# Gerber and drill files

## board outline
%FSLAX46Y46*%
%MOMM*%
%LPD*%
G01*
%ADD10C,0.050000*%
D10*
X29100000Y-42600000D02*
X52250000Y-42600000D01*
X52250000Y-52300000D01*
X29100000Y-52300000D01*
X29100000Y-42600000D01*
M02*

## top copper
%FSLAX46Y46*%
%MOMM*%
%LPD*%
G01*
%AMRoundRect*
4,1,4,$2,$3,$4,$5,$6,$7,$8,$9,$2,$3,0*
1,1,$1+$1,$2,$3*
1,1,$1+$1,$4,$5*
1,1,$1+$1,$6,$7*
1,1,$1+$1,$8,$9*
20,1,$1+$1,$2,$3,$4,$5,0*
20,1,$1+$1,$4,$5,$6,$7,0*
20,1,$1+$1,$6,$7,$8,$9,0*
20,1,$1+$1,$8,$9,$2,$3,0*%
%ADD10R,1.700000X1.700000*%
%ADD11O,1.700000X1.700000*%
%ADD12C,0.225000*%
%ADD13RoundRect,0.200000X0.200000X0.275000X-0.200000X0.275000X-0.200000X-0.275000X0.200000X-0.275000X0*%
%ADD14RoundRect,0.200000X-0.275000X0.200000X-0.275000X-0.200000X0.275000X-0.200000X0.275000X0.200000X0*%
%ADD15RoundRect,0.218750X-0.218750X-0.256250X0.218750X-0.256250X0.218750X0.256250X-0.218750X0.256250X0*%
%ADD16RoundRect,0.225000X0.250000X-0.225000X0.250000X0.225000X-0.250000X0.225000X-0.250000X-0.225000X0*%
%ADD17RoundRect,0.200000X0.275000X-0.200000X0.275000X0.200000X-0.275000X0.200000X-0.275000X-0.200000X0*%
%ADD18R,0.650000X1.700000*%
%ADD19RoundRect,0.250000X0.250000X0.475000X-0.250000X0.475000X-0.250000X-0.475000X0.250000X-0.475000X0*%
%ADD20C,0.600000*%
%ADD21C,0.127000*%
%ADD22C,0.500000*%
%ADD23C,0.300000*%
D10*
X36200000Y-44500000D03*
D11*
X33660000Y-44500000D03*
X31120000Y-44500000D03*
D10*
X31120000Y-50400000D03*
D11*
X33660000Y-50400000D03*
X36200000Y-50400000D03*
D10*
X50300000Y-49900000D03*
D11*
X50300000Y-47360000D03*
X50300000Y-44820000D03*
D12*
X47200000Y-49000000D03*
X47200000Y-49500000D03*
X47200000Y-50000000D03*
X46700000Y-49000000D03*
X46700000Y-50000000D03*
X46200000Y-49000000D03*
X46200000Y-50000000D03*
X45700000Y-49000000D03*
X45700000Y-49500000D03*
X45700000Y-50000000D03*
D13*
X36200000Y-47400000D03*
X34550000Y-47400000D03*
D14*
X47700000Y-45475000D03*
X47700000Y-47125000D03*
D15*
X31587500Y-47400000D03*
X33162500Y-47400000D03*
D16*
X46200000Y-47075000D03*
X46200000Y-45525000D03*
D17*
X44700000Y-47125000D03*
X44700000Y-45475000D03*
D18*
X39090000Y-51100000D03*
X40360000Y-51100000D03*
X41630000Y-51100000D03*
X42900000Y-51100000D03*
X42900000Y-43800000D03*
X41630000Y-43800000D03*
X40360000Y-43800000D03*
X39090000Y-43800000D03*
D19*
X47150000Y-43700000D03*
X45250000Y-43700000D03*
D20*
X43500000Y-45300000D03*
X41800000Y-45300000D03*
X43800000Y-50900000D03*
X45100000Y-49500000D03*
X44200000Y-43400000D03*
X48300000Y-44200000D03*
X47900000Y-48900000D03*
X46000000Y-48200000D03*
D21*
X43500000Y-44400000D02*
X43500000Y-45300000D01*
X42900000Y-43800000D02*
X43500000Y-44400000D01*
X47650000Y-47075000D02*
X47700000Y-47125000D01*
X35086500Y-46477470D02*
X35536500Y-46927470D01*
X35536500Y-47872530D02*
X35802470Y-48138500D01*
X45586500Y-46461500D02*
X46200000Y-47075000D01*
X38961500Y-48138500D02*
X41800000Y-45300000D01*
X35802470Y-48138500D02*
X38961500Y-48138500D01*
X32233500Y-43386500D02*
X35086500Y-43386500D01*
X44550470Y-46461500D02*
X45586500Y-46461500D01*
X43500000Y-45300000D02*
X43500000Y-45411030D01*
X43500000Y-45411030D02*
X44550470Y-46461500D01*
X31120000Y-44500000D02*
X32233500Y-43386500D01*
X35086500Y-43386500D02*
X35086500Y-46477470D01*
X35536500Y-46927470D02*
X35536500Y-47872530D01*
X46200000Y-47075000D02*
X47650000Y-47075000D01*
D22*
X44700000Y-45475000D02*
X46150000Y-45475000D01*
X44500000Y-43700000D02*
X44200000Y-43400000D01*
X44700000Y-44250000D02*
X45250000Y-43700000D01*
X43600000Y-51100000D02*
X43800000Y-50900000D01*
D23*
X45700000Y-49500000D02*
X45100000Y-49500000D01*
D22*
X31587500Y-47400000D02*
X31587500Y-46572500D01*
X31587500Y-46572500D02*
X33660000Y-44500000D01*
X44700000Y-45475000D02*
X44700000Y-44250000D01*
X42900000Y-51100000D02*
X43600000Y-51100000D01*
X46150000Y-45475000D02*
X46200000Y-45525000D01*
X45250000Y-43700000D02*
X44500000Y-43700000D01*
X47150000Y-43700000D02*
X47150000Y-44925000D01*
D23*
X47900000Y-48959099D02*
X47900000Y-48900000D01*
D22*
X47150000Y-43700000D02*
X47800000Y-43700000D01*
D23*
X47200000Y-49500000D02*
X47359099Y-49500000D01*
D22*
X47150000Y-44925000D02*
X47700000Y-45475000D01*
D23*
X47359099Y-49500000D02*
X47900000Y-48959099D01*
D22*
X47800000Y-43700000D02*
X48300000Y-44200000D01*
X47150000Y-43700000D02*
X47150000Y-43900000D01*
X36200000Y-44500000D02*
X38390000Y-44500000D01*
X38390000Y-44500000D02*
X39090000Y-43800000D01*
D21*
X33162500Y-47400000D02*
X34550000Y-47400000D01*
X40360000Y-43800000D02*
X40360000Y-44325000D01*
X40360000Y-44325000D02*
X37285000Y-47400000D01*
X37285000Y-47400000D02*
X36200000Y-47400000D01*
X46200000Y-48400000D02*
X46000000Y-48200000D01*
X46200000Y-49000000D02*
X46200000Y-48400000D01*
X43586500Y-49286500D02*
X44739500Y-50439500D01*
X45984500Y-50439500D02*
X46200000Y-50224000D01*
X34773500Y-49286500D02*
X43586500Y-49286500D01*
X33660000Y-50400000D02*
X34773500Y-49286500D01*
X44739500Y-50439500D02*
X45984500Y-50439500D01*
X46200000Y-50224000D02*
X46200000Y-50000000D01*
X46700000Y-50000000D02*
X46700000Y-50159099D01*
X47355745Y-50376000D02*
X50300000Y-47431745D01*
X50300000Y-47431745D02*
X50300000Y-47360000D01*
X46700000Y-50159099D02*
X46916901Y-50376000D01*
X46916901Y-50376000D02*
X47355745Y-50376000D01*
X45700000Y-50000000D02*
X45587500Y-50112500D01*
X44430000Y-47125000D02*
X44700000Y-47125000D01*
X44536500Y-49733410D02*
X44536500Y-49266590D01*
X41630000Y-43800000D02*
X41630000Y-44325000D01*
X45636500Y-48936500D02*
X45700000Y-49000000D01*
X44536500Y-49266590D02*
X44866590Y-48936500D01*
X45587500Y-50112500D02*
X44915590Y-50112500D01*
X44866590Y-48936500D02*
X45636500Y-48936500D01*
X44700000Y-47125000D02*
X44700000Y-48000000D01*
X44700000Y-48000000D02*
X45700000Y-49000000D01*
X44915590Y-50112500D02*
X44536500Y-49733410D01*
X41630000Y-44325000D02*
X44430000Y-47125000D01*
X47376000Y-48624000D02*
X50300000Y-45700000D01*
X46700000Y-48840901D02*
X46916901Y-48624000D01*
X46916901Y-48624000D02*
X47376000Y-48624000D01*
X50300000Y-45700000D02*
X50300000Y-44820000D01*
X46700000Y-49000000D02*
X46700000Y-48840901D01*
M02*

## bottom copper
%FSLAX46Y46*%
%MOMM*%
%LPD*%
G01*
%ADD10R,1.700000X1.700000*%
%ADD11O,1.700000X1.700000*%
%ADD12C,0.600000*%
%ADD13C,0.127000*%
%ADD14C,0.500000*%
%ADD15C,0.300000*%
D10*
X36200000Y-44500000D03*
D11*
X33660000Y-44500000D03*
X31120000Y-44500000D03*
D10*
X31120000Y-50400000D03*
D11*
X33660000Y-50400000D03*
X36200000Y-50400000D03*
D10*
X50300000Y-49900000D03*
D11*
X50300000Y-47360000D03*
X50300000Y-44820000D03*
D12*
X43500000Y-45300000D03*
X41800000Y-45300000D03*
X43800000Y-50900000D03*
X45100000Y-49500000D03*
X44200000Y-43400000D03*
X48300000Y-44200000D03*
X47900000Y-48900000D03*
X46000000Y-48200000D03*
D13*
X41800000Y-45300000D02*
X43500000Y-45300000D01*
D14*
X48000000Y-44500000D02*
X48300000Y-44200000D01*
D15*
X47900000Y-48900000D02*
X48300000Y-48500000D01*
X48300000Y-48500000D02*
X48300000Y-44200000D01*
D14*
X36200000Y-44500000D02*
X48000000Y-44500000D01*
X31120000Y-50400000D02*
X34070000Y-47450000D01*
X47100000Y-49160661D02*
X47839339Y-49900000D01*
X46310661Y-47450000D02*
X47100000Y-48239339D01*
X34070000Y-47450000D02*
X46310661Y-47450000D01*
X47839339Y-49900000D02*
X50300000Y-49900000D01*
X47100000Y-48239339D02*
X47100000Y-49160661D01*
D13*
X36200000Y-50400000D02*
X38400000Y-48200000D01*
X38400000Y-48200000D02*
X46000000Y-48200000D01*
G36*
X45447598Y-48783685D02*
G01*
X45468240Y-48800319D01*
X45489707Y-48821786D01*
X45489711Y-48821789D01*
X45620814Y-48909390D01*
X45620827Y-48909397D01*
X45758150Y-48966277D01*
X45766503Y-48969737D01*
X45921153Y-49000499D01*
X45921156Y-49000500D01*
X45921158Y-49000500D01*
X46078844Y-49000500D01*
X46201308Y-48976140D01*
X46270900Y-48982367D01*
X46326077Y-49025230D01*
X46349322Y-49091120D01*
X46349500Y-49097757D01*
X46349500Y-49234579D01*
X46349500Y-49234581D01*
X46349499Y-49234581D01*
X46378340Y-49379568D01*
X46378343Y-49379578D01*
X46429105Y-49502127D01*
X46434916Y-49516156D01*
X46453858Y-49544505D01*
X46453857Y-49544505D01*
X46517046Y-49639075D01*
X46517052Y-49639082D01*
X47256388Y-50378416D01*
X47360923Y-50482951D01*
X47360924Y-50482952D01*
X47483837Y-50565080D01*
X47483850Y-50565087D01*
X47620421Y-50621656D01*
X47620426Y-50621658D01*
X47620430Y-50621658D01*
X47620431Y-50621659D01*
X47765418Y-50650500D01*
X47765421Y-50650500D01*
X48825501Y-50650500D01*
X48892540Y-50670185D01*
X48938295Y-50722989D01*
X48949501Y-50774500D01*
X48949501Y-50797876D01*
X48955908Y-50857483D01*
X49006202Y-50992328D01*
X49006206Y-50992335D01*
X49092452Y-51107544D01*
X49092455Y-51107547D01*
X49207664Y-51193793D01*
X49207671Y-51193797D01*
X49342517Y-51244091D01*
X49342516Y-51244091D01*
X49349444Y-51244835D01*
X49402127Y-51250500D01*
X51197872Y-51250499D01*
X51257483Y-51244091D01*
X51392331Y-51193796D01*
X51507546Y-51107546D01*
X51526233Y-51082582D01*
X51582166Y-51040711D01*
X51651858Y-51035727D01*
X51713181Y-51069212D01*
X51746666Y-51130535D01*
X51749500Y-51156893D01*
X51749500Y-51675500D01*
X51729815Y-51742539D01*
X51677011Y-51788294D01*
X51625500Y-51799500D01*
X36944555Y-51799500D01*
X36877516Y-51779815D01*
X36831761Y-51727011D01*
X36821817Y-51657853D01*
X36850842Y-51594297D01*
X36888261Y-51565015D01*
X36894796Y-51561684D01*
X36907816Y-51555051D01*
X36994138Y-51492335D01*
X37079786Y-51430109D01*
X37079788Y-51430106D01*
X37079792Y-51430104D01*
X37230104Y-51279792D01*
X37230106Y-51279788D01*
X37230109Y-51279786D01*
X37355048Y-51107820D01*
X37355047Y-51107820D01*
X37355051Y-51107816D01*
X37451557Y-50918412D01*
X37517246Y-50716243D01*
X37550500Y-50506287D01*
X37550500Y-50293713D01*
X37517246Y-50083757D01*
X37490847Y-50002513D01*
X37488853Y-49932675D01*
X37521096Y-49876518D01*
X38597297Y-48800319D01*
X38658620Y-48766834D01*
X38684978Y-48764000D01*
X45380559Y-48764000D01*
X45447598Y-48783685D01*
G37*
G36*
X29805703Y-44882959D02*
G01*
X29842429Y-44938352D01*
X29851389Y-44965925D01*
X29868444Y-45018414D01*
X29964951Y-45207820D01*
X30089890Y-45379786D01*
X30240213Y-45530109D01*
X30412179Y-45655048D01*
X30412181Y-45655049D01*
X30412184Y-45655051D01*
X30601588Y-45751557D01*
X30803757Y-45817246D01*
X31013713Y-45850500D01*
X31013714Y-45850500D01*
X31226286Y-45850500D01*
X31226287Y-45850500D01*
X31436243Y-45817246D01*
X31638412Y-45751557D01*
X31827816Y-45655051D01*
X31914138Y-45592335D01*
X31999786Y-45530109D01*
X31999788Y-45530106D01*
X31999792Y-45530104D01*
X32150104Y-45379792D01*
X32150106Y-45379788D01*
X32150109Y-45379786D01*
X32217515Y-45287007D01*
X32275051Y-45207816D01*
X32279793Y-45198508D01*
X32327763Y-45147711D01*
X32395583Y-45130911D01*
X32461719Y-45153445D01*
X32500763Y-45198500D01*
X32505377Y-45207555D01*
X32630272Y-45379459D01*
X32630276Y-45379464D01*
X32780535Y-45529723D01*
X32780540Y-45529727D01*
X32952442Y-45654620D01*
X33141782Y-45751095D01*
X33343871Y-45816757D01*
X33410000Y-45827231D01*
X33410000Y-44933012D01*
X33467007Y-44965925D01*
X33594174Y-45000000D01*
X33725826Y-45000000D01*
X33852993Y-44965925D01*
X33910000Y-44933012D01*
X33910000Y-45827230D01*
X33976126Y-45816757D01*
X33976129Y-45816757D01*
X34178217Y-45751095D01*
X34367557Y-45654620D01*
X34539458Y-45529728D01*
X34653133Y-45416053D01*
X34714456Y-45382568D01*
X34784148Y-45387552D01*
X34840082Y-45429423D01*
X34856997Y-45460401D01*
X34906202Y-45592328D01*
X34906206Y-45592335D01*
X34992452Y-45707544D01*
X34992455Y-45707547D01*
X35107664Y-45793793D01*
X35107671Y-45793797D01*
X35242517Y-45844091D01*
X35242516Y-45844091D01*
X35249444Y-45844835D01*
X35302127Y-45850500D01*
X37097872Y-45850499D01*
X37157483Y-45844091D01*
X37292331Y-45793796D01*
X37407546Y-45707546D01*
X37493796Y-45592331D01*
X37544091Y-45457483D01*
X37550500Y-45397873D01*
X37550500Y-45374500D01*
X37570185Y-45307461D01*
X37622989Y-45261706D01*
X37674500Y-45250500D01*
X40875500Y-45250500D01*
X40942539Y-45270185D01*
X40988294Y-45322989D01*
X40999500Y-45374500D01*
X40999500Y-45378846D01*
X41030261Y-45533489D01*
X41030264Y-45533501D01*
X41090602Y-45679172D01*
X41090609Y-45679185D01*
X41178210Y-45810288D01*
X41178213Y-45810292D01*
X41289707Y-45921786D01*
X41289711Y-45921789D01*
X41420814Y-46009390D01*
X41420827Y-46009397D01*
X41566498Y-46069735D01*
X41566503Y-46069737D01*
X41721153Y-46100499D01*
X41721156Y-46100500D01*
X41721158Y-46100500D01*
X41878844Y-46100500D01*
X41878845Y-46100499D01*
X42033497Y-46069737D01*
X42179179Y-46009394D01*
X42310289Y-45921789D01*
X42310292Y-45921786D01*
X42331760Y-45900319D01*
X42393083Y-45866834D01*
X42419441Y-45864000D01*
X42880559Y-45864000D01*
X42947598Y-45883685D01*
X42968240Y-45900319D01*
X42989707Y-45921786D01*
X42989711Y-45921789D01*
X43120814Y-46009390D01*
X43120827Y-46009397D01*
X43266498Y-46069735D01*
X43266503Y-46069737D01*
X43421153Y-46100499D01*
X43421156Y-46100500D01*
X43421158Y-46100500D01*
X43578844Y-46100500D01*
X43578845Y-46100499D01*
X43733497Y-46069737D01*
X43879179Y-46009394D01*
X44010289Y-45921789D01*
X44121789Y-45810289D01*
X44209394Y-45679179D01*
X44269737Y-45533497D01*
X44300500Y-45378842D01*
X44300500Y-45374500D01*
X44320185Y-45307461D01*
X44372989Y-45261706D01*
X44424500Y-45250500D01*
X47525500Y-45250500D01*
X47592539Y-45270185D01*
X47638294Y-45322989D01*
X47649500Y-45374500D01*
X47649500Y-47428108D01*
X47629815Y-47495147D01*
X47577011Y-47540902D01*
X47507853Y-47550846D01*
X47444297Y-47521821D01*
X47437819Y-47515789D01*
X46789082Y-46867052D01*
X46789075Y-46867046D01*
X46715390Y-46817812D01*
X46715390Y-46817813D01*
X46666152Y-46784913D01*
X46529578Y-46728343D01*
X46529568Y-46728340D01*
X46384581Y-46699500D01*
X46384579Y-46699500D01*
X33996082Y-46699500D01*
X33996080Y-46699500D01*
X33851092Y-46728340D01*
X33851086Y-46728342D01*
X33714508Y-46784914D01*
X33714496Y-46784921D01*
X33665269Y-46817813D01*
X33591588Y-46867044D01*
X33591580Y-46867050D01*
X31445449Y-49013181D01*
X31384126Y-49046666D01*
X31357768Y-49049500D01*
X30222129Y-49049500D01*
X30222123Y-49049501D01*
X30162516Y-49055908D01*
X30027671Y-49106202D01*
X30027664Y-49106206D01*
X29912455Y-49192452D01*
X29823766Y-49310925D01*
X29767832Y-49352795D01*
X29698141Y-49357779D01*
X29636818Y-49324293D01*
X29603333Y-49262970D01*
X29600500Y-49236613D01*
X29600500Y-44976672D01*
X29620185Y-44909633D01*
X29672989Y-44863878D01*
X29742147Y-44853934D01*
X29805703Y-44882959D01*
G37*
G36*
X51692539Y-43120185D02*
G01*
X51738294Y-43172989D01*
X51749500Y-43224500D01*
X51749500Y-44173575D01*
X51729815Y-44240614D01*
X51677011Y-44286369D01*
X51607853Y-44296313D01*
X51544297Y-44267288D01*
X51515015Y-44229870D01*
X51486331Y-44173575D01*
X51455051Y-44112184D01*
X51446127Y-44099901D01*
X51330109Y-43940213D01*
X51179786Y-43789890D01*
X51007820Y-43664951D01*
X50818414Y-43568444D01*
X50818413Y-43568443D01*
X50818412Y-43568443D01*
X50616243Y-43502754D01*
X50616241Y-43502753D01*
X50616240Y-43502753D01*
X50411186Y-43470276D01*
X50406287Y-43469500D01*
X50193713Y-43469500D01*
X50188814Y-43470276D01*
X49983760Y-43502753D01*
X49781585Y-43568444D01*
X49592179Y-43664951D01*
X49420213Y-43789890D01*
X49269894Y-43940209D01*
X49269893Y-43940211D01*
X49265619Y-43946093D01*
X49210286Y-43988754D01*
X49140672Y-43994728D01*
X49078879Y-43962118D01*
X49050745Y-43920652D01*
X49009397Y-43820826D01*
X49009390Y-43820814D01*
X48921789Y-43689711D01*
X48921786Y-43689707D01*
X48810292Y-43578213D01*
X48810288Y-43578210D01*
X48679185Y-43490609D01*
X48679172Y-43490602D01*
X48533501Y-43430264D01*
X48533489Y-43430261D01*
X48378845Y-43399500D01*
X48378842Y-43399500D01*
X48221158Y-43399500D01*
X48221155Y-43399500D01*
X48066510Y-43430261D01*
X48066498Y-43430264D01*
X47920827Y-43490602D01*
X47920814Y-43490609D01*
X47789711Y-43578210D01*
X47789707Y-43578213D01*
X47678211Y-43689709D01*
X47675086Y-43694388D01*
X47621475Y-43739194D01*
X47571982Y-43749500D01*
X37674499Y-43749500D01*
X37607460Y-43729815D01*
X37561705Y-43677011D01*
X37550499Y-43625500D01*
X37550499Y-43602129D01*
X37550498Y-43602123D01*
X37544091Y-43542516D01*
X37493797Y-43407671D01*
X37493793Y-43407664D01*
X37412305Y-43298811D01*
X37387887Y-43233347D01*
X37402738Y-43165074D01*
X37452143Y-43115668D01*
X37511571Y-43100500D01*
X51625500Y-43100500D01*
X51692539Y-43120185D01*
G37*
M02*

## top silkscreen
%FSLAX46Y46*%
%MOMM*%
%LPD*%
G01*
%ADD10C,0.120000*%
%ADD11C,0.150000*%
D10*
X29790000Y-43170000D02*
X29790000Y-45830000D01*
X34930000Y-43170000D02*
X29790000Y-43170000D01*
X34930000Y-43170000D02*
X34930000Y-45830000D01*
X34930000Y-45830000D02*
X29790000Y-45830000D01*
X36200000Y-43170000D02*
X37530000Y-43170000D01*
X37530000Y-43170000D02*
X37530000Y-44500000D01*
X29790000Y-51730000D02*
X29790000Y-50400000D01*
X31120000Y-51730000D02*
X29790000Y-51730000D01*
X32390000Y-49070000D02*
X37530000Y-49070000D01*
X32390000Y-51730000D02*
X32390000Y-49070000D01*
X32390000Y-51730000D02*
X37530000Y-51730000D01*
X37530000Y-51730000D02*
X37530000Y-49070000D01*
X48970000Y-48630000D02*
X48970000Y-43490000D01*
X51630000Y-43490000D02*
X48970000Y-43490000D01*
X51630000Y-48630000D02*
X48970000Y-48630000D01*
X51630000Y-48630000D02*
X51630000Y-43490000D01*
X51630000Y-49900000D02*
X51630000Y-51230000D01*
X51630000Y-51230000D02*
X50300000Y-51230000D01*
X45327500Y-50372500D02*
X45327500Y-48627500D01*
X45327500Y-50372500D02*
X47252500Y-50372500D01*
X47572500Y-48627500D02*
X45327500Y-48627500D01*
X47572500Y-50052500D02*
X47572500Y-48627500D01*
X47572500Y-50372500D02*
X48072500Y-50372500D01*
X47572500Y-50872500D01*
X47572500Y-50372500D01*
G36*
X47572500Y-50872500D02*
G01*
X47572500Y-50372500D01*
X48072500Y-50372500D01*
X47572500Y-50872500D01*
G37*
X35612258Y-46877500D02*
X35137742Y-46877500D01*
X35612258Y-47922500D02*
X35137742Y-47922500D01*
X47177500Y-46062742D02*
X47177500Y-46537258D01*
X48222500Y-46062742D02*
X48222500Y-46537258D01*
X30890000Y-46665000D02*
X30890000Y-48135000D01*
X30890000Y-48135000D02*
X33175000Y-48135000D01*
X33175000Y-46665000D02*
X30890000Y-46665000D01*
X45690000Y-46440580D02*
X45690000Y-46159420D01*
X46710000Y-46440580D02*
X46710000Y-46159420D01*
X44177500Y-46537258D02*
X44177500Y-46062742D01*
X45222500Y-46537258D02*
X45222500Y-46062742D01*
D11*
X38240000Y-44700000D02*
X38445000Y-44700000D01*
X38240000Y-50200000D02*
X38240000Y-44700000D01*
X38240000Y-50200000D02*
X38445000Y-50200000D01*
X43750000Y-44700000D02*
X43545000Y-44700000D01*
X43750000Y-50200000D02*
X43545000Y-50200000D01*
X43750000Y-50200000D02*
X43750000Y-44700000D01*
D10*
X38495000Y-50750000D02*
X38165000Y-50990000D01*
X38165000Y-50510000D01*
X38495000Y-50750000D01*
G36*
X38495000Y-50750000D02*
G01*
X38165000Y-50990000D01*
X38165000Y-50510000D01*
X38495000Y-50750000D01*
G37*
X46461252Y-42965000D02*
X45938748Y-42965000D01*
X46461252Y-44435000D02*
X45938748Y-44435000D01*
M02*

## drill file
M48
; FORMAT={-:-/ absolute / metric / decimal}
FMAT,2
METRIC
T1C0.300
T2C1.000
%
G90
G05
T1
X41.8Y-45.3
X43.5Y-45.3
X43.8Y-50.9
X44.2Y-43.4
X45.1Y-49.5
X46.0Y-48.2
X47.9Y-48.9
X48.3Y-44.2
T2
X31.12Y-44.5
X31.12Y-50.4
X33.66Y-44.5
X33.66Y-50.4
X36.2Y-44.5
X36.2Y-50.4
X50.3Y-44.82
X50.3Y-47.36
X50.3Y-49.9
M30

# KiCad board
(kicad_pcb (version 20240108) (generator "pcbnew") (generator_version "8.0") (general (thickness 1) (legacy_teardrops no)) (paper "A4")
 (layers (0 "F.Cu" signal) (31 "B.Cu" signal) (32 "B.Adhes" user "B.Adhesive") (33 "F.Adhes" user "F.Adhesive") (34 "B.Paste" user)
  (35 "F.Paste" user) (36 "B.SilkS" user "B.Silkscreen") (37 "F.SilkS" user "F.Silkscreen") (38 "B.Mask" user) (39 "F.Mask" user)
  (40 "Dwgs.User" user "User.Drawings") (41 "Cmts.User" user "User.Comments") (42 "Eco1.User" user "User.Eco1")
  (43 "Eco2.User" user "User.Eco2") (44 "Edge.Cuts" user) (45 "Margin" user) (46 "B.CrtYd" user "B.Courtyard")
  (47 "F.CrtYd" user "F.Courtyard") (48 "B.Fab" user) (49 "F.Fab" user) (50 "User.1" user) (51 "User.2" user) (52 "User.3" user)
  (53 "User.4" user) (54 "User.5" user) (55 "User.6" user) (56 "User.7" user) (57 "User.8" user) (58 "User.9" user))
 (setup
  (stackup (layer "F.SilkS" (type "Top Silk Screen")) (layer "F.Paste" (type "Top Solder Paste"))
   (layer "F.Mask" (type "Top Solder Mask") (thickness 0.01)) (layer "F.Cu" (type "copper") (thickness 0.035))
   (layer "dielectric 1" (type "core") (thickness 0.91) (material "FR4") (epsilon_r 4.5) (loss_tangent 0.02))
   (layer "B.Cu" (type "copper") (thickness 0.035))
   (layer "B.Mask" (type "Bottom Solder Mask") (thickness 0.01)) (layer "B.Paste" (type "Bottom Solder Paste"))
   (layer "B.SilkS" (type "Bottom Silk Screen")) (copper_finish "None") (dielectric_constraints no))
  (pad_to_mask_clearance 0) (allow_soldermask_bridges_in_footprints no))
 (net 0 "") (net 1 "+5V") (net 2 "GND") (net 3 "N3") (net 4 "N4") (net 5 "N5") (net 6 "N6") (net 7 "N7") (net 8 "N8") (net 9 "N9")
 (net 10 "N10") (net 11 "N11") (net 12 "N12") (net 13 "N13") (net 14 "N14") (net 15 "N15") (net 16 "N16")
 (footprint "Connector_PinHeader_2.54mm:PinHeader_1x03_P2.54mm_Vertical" (layer "F.Cu") (at 36.2 44.5 -90)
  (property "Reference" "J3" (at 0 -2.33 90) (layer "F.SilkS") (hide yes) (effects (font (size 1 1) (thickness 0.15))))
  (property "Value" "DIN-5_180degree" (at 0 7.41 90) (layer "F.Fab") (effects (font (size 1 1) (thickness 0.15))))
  (fp_line (start -1.33 6.41) (end 1.33 6.41) (stroke (width 0.12) (type solid)) (layer "F.SilkS"))
  (fp_line (start -1.33 1.27) (end -1.33 6.41) (stroke (width 0.12) (type solid)) (layer "F.SilkS"))
  (fp_line (start -1.33 1.27) (end 1.33 1.27) (stroke (width 0.12) (type solid)) (layer "F.SilkS"))
  (fp_line (start 1.33 1.27) (end 1.33 6.41) (stroke (width 0.12) (type solid)) (layer "F.SilkS"))
  (fp_line (start -1.33 0) (end -1.33 -1.33) (stroke (width 0.12) (type solid)) (layer "F.SilkS"))
  (fp_line (start -1.33 -1.33) (end 0 -1.33) (stroke (width 0.12) (type solid)) (layer "F.SilkS"))
  (pad "1" thru_hole rect (at 0 0 270) (size 1.7 1.7) (drill 1) (layers "*.Cu" "*.Mask") (remove_unused_layers no) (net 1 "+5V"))
  (pad "2" thru_hole oval (at 0 2.54 270) (size 1.7 1.7) (drill 1) (layers "*.Cu" "*.Mask") (remove_unused_layers no) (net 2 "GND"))
  (pad "3" thru_hole oval (at 0 5.08 270) (size 1.7 1.7) (drill 1) (layers "*.Cu" "*.Mask") (remove_unused_layers no) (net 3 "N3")))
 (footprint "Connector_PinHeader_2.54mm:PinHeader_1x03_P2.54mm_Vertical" (layer "F.Cu") (at 31.12 50.4 90)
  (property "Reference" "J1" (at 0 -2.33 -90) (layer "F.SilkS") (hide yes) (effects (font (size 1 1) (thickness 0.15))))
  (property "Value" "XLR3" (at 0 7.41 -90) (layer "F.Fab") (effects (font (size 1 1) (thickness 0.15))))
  (fp_line (start -1.33 -1.33) (end 0 -1.33) (stroke (width 0.12) (type solid)) (layer "F.SilkS"))
  (fp_line (start -1.33 0) (end -1.33 -1.33) (stroke (width 0.12) (type solid)) (layer "F.SilkS"))
  (fp_line (start 1.33 1.27) (end 1.33 6.41) (stroke (width 0.12) (type solid)) (layer "F.SilkS"))
  (fp_line (start -1.33 1.27) (end 1.33 1.27) (stroke (width 0.12) (type solid)) (layer "F.SilkS"))
  (fp_line (start -1.33 1.27) (end -1.33 6.41) (stroke (width 0.12) (type solid)) (layer "F.SilkS"))
  (fp_line (start -1.33 6.41) (end 1.33 6.41) (stroke (width 0.12) (type solid)) (layer "F.SilkS"))
  (pad "1" thru_hole rect (at 0 0 90) (size 1.7 1.7) (drill 1) (layers "*.Cu" "*.Mask") (remove_unused_layers no) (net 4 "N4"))
  (pad "2" thru_hole oval (at 0 2.54 90) (size 1.7 1.7) (drill 1) (layers "*.Cu" "*.Mask") (remove_unused_layers no) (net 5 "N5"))
  (pad "3" thru_hole oval (at 0 5.08 90) (size 1.7 1.7) (drill 1) (layers "*.Cu" "*.Mask") (remove_unused_layers no) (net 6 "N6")))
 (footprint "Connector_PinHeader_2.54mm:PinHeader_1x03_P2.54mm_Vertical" (layer "F.Cu") (at 50.3 49.9 180)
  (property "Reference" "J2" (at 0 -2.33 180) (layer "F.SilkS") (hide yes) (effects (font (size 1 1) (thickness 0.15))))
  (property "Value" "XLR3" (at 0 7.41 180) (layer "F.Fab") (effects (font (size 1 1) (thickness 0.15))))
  (fp_line (start 1.33 1.27) (end 1.33 6.41) (stroke (width 0.12) (type solid)) (layer "F.SilkS"))
  (fp_line (start -1.33 6.41) (end 1.33 6.41) (stroke (width 0.12) (type solid)) (layer "F.SilkS"))
  (fp_line (start -1.33 1.27) (end 1.33 1.27) (stroke (width 0.12) (type solid)) (layer "F.SilkS"))
  (fp_line (start -1.33 1.27) (end -1.33 6.41) (stroke (width 0.12) (type solid)) (layer "F.SilkS"))
  (fp_line (start -1.33 0) (end -1.33 -1.33) (stroke (width 0.12) (type solid)) (layer "F.SilkS"))
  (fp_line (start -1.33 -1.33) (end 0 -1.33) (stroke (width 0.12) (type solid)) (layer "F.SilkS"))
  (pad "1" thru_hole rect (at 0 0 180) (size 1.7 1.7) (drill 1) (layers "*.Cu" "*.Mask") (remove_unused_layers no) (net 4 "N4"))
  (pad "2" thru_hole oval (at 0 2.54 180) (size 1.7 1.7) (drill 1) (layers "*.Cu" "*.Mask") (remove_unused_layers no) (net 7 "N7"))
  (pad "3" thru_hole oval (at 0 5.08 180) (size 1.7 1.7) (drill 1) (layers "*.Cu" "*.Mask") (remove_unused_layers no) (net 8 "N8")))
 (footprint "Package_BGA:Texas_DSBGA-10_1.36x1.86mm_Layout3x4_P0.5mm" (layer "F.Cu") (at 46.45 49.5 -90)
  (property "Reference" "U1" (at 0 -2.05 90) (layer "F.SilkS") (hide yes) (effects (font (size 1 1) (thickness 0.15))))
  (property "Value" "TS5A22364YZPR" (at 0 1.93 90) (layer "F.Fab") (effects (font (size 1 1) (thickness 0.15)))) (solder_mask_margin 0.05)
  (fp_line (start 0.8725 1.1225) (end -0.8725 1.1225) (stroke (width 0.12) (type solid)) (layer "F.SilkS"))
  (fp_line (start 0.8725 1.1225) (end 0.8725 -0.8025) (stroke (width 0.12) (type solid)) (layer "F.SilkS"))
  (fp_line (start -0.8725 -1.1225) (end -0.8725 1.1225) (stroke (width 0.12) (type solid)) (layer "F.SilkS"))
  (fp_line (start 0.5525 -1.1225) (end -0.8725 -1.1225) (stroke (width 0.12) (type solid)) (layer "F.SilkS"))
  (fp_poly
   (pts (xy 0.8725 -1.1225) (xy 0.8725 -1.6225) (xy 1.3725 -1.1225) (xy 0.8725 -1.1225)) (stroke (width 0.12) (type solid)) (fill solid)
   (layer "F.SilkS"))
  (pad "" smd roundrect (at -0.5 -0.75 270) (size 0.25 0.25) (layers "F.Paste") (roundrect_rratio 0.2))
  (pad "" smd roundrect (at -0.5 -0.25 270) (size 0.25 0.25) (layers "F.Paste") (roundrect_rratio 0.2))
  (pad "" smd roundrect (at -0.5 0.25 270) (size 0.25 0.25) (layers "F.Paste") (roundrect_rratio 0.2))
  (pad "" smd roundrect (at -0.5 0.75 270) (size 0.25 0.25) (layers "F.Paste") (roundrect_rratio 0.2))
  (pad "" smd roundrect (at 0 -0.75 270) (size 0.25 0.25) (layers "F.Paste") (roundrect_rratio 0.2))
  (pad "" smd roundrect (at 0 0.75 270) (size 0.25 0.25) (layers "F.Paste") (roundrect_rratio 0.2))
  (pad "" smd roundrect (at 0.5 -0.75 270) (size 0.25 0.25) (layers "F.Paste") (roundrect_rratio 0.2))
  (pad "" smd roundrect (at 0.5 -0.25 270) (size 0.25 0.25) (layers "F.Paste") (roundrect_rratio 0.2))
  (pad "" smd roundrect (at 0.5 0.25 270) (size 0.25 0.25) (layers "F.Paste") (roundrect_rratio 0.2))
  (pad "" smd roundrect (at 0.5 0.75 270) (size 0.25 0.25) (layers "F.Paste") (roundrect_rratio 0.2))
  (pad "A1" smd circle (at -0.5 -0.75 270) (size 0.225 0.225) (layers "F.Cu" "F.Mask") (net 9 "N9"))
  (pad "A2" smd circle (at 0 -0.75 270) (size 0.225 0.225) (layers "F.Cu" "F.Mask") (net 1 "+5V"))
  (pad "A3" smd circle (at 0.5 -0.75 270) (size 0.225 0.225) (layers "F.Cu" "F.Mask") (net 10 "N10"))
  (pad "B1" smd circle (at -0.5 -0.25 270) (size 0.225 0.225) (layers "F.Cu" "F.Mask") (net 8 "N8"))
  (pad "B3" smd circle (at 0.5 -0.25 270) (size 0.225 0.225) (layers "F.Cu" "F.Mask") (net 7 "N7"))
  (pad "C1" smd circle (at -0.5 0.25 270) (size 0.225 0.225) (layers "F.Cu" "F.Mask") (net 6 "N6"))
  (pad "C3" smd circle (at 0.5 0.25 270) (size 0.225 0.225) (layers "F.Cu" "F.Mask") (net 5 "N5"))
  (pad "D1" smd circle (at -0.5 0.75 270) (size 0.225 0.225) (layers "F.Cu" "F.Mask") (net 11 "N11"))
  (pad "D2" smd circle (at 0 0.75 270) (size 0.225 0.225) (layers "F.Cu" "F.Mask") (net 2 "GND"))
  (pad "D3" smd circle (at 0.5 0.75 270) (size 0.225 0.225) (layers "F.Cu" "F.Mask") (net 11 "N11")))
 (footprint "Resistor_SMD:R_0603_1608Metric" (layer "F.Cu") (at 35.375 47.4 180)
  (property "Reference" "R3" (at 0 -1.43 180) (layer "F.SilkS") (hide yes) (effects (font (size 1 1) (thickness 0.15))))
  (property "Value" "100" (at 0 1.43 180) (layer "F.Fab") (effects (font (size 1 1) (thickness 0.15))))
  (fp_line (start -0.237258 0.5225) (end 0.237258 0.5225) (stroke (width 0.12) (type solid)) (layer "F.SilkS"))
  (fp_line (start -0.237258 -0.5225) (end 0.237258 -0.5225) (stroke (width 0.12) (type solid)) (layer "F.SilkS"))
  (pad "1" smd roundrect (at -0.825 0 180) (size 0.8 0.95) (layers "F.Cu" "F.Paste" "F.Mask") (roundrect_rratio 0.25) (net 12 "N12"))
  (pad "2" smd roundrect (at 0.825 0 180) (size 0.8 0.95) (layers "F.Cu" "F.Paste" "F.Mask") (roundrect_rratio 0.25) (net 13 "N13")))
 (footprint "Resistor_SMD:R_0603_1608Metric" (layer "F.Cu") (at 47.7 46.3 -90)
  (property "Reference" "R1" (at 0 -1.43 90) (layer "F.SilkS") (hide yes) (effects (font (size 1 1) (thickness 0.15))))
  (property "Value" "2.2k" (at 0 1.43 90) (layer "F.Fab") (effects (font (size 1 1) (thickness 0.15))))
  (fp_line (start -0.237258 0.5225) (end 0.237258 0.5225) (stroke (width 0.12) (type solid)) (layer "F.SilkS"))
  (fp_line (start -0.237258 -0.5225) (end 0.237258 -0.5225) (stroke (width 0.12) (type solid)) (layer "F.SilkS"))
  (pad "1" smd roundrect (at -0.825 0 270) (size 0.8 0.95) (layers "F.Cu" "F.Paste" "F.Mask") (roundrect_rratio 0.25) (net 1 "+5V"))
  (pad "2" smd roundrect (at 0.825 0 270) (size 0.8 0.95) (layers "F.Cu" "F.Paste" "F.Mask") (roundrect_rratio 0.25) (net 3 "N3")))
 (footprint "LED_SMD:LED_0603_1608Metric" (layer "F.Cu") (at 32.375 47.4)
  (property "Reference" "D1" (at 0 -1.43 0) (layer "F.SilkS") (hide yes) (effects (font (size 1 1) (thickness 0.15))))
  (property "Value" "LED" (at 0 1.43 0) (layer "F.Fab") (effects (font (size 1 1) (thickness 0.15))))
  (fp_line (start -1.485 -0.735) (end -1.485 0.735) (stroke (width 0.12) (type solid)) (layer "F.SilkS"))
  (fp_line (start -1.485 0.735) (end 0.8 0.735) (stroke (width 0.12) (type solid)) (layer "F.SilkS"))
  (fp_line (start 0.8 -0.735) (end -1.485 -0.735) (stroke (width 0.12) (type solid)) (layer "F.SilkS"))
  (pad "1" smd roundrect (at -0.7875 0) (size 0.875 0.95) (layers "F.Cu" "F.Paste" "F.Mask") (roundrect_rratio 0.25) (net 2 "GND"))
  (pad "2" smd roundrect (at 0.7875 0) (size 0.875 0.95) (layers "F.Cu" "F.Paste" "F.Mask") (roundrect_rratio 0.25) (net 13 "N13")))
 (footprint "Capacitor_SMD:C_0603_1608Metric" (layer "F.Cu") (at 46.2 46.3 90)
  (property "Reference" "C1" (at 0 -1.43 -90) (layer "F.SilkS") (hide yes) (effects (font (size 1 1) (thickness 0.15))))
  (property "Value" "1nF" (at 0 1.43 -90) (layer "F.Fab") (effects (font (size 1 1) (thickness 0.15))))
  (fp_line (start -0.14058 -0.51) (end 0.14058 -0.51) (stroke (width 0.12) (type solid)) (layer "F.SilkS"))
  (fp_line (start -0.14058 0.51) (end 0.14058 0.51) (stroke (width 0.12) (type solid)) (layer "F.SilkS"))
  (pad "1" smd roundrect (at -0.775 0 90) (size 0.9 0.95) (layers "F.Cu" "F.Paste" "F.Mask") (roundrect_rratio 0.25) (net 3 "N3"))
  (pad "2" smd roundrect (at 0.775 0 90) (size 0.9 0.95) (layers "F.Cu" "F.Paste" "F.Mask") (roundrect_rratio 0.25) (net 2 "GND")))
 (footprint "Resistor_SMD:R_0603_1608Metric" (layer "F.Cu") (at 44.7 46.3 90)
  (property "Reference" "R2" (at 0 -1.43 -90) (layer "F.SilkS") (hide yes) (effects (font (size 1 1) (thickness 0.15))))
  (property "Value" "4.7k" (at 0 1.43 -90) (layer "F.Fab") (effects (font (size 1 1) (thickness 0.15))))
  (fp_line (start -0.237258 -0.5225) (end 0.237258 -0.5225) (stroke (width 0.12) (type solid)) (layer "F.SilkS"))
  (fp_line (start -0.237258 0.5225) (end 0.237258 0.5225) (stroke (width 0.12) (type solid)) (layer "F.SilkS"))
  (pad "1" smd roundrect (at -0.825 0 90) (size 0.8 0.95) (layers "F.Cu" "F.Paste" "F.Mask") (roundrect_rratio 0.25) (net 11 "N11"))
  (pad "2" smd roundrect (at 0.825 0 90) (size 0.8 0.95) (layers "F.Cu" "F.Paste" "F.Mask") (roundrect_rratio 0.25) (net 2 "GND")))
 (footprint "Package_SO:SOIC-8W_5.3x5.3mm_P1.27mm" (layer "F.Cu") (at 40.995 47.45 90)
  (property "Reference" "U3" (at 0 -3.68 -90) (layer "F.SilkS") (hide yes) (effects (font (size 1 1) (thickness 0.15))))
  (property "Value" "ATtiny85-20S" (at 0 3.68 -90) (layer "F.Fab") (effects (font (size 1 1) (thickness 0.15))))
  (fp_line (start 2.75 -2.755) (end 2.75 -2.55) (stroke (width 0.15) (type solid)) (layer "F.SilkS"))
  (fp_line (start -2.75 -2.755) (end 2.75 -2.755) (stroke (width 0.15) (type solid)) (layer "F.SilkS"))
  (fp_line (start -2.75 -2.755) (end -2.75 -2.55) (stroke (width 0.15) (type solid)) (layer "F.SilkS"))
  (fp_line (start 2.75 2.755) (end 2.75 2.55) (stroke (width 0.15) (type solid)) (layer "F.SilkS"))
  (fp_line (start -2.75 2.755) (end -2.75 2.55) (stroke (width 0.15) (type solid)) (layer "F.SilkS"))
  (fp_line (start -2.75 2.755) (end 2.75 2.755) (stroke (width 0.15) (type solid)) (layer "F.SilkS"))
  (fp_poly
   (pts (xy -3.3 -2.5) (xy -3.54 -2.83) (xy -3.06 -2.83) (xy -3.3 -2.5)) (stroke (width 0.12) (type solid)) (fill solid) (layer "F.SilkS"))
  (pad "1" smd rect (at -3.65 -1.905 90) (size 1.7 0.65) (layers "F.Cu" "F.Paste" "F.Mask") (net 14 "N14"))
  (pad "2" smd rect (at -3.65 -0.635 90) (size 1.7 0.65) (layers "F.Cu" "F.Paste" "F.Mask") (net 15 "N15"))
  (pad "3" smd rect (at -3.65 0.635 90) (size 1.7 0.65) (layers "F.Cu" "F.Paste" "F.Mask") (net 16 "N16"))
  (pad "4" smd rect (at -3.65 1.905 90) (size 1.7 0.65) (layers "F.Cu" "F.Paste" "F.Mask") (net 2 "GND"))
  (pad "5" smd rect (at 3.65 1.905 90) (size 1.7 0.65) (layers "F.Cu" "F.Paste" "F.Mask") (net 3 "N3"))
  (pad "6" smd rect (at 3.65 0.635 90) (size 1.7 0.65) (layers "F.Cu" "F.Paste" "F.Mask") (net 11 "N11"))
  (pad "7" smd rect (at 3.65 -0.635 90) (size 1.7 0.65) (layers "F.Cu" "F.Paste" "F.Mask") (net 12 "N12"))
  (pad "8" smd rect (at 3.65 -1.905 90) (size 1.7 0.65) (layers "F.Cu" "F.Paste" "F.Mask") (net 1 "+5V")))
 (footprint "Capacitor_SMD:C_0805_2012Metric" (layer "F.Cu") (at 46.2 43.7 180)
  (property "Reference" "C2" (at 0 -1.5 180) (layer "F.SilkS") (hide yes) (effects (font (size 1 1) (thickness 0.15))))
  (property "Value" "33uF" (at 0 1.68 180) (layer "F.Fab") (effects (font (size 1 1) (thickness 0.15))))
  (fp_line (start -0.261252 0.735) (end 0.261252 0.735) (stroke (width 0.12) (type solid)) (layer "F.SilkS"))
  (fp_line (start -0.261252 -0.735) (end 0.261252 -0.735) (stroke (width 0.12) (type solid)) (layer "F.SilkS"))
  (pad "1" smd roundrect (at -0.95 0 180) (size 1 1.45) (layers "F.Cu" "F.Paste" "F.Mask") (roundrect_rratio 0.25) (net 1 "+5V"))
  (pad "2" smd roundrect (at 0.95 0 180) (size 1 1.45) (layers "F.Cu" "F.Paste" "F.Mask") (roundrect_rratio 0.25) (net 2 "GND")))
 (gr_rect (start 29.1 42.6) (end 52.25 52.3) (stroke (width 0.05) (type default)) (fill none) (layer "Edge.Cuts"))
 (segment (start 43.5 44.4) (end 43.5 45.3) (width 0.127) (layer "F.Cu") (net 3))
 (segment (start 42.9 43.8) (end 43.5 44.4) (width 0.127) (layer "F.Cu") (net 3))
 (segment (start 47.65 47.075) (end 47.7 47.125) (width 0.127) (layer "F.Cu") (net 3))
 (segment (start 35.0865 46.47747) (end 35.5365 46.92747) (width 0.127) (layer "F.Cu") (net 3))
 (segment (start 35.5365 47.87253) (end 35.80247 48.1385) (width 0.127) (layer "F.Cu") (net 3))
 (segment (start 45.5865 46.4615) (end 46.2 47.075) (width 0.127) (layer "F.Cu") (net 3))
 (segment (start 38.9615 48.1385) (end 41.8 45.3) (width 0.127) (layer "F.Cu") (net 3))
 (segment (start 35.80247 48.1385) (end 38.9615 48.1385) (width 0.127) (layer "F.Cu") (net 3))
 (segment (start 32.2335 43.3865) (end 35.0865 43.3865) (width 0.127) (layer "F.Cu") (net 3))
 (segment (start 44.55047 46.4615) (end 45.5865 46.4615) (width 0.127) (layer "F.Cu") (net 3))
 (segment (start 43.5 45.3) (end 43.5 45.41103) (width 0.127) (layer "F.Cu") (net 3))
 (segment (start 43.5 45.41103) (end 44.55047 46.4615) (width 0.127) (layer "F.Cu") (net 3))
 (segment (start 31.12 44.5) (end 32.2335 43.3865) (width 0.127) (layer "F.Cu") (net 3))
 (segment (start 35.0865 43.3865) (end 35.0865 46.47747) (width 0.127) (layer "F.Cu") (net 3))
 (segment (start 35.5365 46.92747) (end 35.5365 47.87253) (width 0.127) (layer "F.Cu") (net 3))
 (segment (start 46.2 47.075) (end 47.65 47.075) (width 0.127) (layer "F.Cu") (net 3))
 (via (at 43.5 45.3) (size 0.6) (drill 0.3) (layers "F.Cu" "B.Cu") (free yes) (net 3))
 (via (at 41.8 45.3) (size 0.6) (drill 0.3) (layers "F.Cu" "B.Cu") (free yes) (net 3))
 (segment (start 41.8 45.3) (end 43.5 45.3) (width 0.127) (layer "B.Cu") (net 3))
 (segment (start 44.7 45.475) (end 46.15 45.475) (width 0.5) (layer "F.Cu") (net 2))
 (segment (start 44.5 43.7) (end 44.2 43.4) (width 0.5) (layer "F.Cu") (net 2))
 (segment (start 44.7 44.25) (end 45.25 43.7) (width 0.5) (layer "F.Cu") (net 2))
 (segment (start 43.6 51.1) (end 43.8 50.9) (width 0.5) (layer "F.Cu") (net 2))
 (segment (start 45.7 49.5) (end 45.1 49.5) (width 0.3) (layer "F.Cu") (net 2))
 (segment (start 31.5875 47.4) (end 31.5875 46.5725) (width 0.5) (layer "F.Cu") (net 2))
 (segment (start 31.5875 46.5725) (end 33.66 44.5) (width 0.5) (layer "F.Cu") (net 2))
 (segment (start 44.7 45.475) (end 44.7 44.25) (width 0.5) (layer "F.Cu") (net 2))
 (segment (start 42.9 51.1) (end 43.6 51.1) (width 0.5) (layer "F.Cu") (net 2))
 (segment (start 46.15 45.475) (end 46.2 45.525) (width 0.5) (layer "F.Cu") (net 2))
 (segment (start 45.25 43.7) (end 44.5 43.7) (width 0.5) (layer "F.Cu") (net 2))
 (via (at 43.8 50.9) (size 0.6) (drill 0.3) (layers "F.Cu" "B.Cu") (free yes) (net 2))
 (via (at 45.1 49.5) (size 0.6) (drill 0.3) (layers "F.Cu" "B.Cu") (free yes) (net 2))
 (via (at 44.2 43.4) (size 0.6) (drill 0.3) (layers "F.Cu" "B.Cu") (free yes) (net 2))
 (segment (start 47.15 43.7) (end 47.15 44.925) (width 0.5) (layer "F.Cu") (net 1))
 (segment (start 47.9 48.959099) (end 47.9 48.9) (width 0.3) (layer "F.Cu") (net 1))
 (segment (start 47.15 43.7) (end 47.8 43.7) (width 0.5) (layer "F.Cu") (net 1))
 (segment (start 47.2 49.5) (end 47.359099 49.5) (width 0.3) (layer "F.Cu") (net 1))
 (segment (start 47.15 44.925) (end 47.7 45.475) (width 0.5) (layer "F.Cu") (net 1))
 (segment (start 47.359099 49.5) (end 47.9 48.959099) (width 0.3) (layer "F.Cu") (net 1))
 (segment (start 47.8 43.7) (end 48.3 44.2) (width 0.5) (layer "F.Cu") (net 1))
 (segment (start 47.15 43.7) (end 47.15 43.9) (width 0.5) (layer "F.Cu") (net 1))
 (segment (start 36.2 44.5) (end 38.39 44.5) (width 0.5) (layer "F.Cu") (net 1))
 (segment (start 38.39 44.5) (end 39.09 43.8) (width 0.5) (layer "F.Cu") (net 1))
 (via (at 48.3 44.2) (size 0.6) (drill 0.3) (layers "F.Cu" "B.Cu") (free yes) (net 1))
 (via (at 47.9 48.9) (size 0.6) (drill 0.3) (layers "F.Cu" "B.Cu") (free yes) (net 1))
 (segment (start 48 44.5) (end 48.3 44.2) (width 0.5) (layer "B.Cu") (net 1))
 (segment (start 47.9 48.9) (end 48.3 48.5) (width 0.3) (layer "B.Cu") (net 1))
 (segment (start 48.3 48.5) (end 48.3 44.2) (width 0.3) (layer "B.Cu") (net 1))
 (segment (start 36.2 44.5) (end 48 44.5) (width 0.5) (layer "B.Cu") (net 1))
 (segment (start 33.1625 47.4) (end 34.55 47.4) (width 0.127) (layer "F.Cu") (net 13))
 (segment (start 31.12 50.4) (end 34.07 47.45) (width 0.5) (layer "B.Cu") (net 4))
 (segment (start 47.1 49.160661) (end 47.839339 49.9) (width 0.5) (layer "B.Cu") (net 4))
 (segment (start 46.310661 47.45) (end 47.1 48.239339) (width 0.5) (layer "B.Cu") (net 4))
 (segment (start 34.07 47.45) (end 46.310661 47.45) (width 0.5) (layer "B.Cu") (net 4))
 (segment (start 47.839339 49.9) (end 50.3 49.9) (width 0.5) (layer "B.Cu") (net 4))
 (segment (start 47.1 48.239339) (end 47.1 49.160661) (width 0.5) (layer "B.Cu") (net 4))
 (segment (start 40.36 43.8) (end 40.36 44.325) (width 0.127) (layer "F.Cu") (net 12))
 (segment (start 40.36 44.325) (end 37.285 47.4) (width 0.127) (layer "F.Cu") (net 12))
 (segment (start 37.285 47.4) (end 36.2 47.4) (width 0.127) (layer "F.Cu") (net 12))
 (segment (start 46.2 48.4) (end 46 48.2) (width 0.127) (layer "F.Cu") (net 6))
 (segment (start 46.2 49) (end 46.2 48.4) (width 0.127) (layer "F.Cu") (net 6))
 (via (at 46 48.2) (size 0.6) (drill 0.3) (layers "F.Cu" "B.Cu") (free yes) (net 6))
 (segment (start 36.2 50.4) (end 38.4 48.2) (width 0.127) (layer "B.Cu") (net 6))
 (segment (start 38.4 48.2) (end 46 48.2) (width 0.127) (layer "B.Cu") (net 6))
 (segment (start 43.5865 49.2865) (end 44.7395 50.4395) (width 0.127) (layer "F.Cu") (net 5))
 (segment (start 45.9845 50.4395) (end 46.2 50.224) (width 0.127) (layer "F.Cu") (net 5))
 (segment (start 34.7735 49.2865) (end 43.5865 49.2865) (width 0.127) (layer "F.Cu") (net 5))
 (segment (start 33.66 50.4) (end 34.7735 49.2865) (width 0.127) (layer "F.Cu") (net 5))
 (segment (start 44.7395 50.4395) (end 45.9845 50.4395) (width 0.127) (layer "F.Cu") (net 5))
 (segment (start 46.2 50.224) (end 46.2 50) (width 0.127) (layer "F.Cu") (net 5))
 (segment (start 46.7 50) (end 46.7 50.159099) (width 0.127) (layer "F.Cu") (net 7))
 (segment (start 47.355745 50.376) (end 50.3 47.431745) (width 0.127) (layer "F.Cu") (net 7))
 (segment (start 50.3 47.431745) (end 50.3 47.36) (width 0.127) (layer "F.Cu") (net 7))
 (segment (start 46.7 50.159099) (end 46.916901 50.376) (width 0.127) (layer "F.Cu") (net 7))
 (segment (start 46.916901 50.376) (end 47.355745 50.376) (width 0.127) (layer "F.Cu") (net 7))
 (segment (start 45.7 50) (end 45.5875 50.1125) (width 0.127) (layer "F.Cu") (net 11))
 (segment (start 44.43 47.125) (end 44.7 47.125) (width 0.127) (layer "F.Cu") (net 11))
 (segment (start 44.5365 49.73341) (end 44.5365 49.26659) (width 0.127) (layer "F.Cu") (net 11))
 (segment (start 41.63 43.8) (end 41.63 44.325) (width 0.127) (layer "F.Cu") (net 11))
 (segment (start 45.6365 48.9365) (end 45.7 49) (width 0.127) (layer "F.Cu") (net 11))
 (segment (start 44.5365 49.26659) (end 44.86659 48.9365) (width 0.127) (layer "F.Cu") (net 11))
 (segment (start 45.5875 50.1125) (end 44.91559 50.1125) (width 0.127) (layer "F.Cu") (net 11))
 (segment (start 44.86659 48.9365) (end 45.6365 48.9365) (width 0.127) (layer "F.Cu") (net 11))
 (segment (start 44.7 47.125) (end 44.7 48) (width 0.127) (layer "F.Cu") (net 11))
 (segment (start 44.7 48) (end 45.7 49) (width 0.127) (layer "F.Cu") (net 11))
 (segment (start 44.91559 50.1125) (end 44.5365 49.73341) (width 0.127) (layer "F.Cu") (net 11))
 (segment (start 41.63 44.325) (end 44.43 47.125) (width 0.127) (layer "F.Cu") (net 11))
 (segment (start 47.376 48.624) (end 50.3 45.7) (width 0.127) (layer "F.Cu") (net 8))
 (segment (start 46.7 48.840901) (end 46.916901 48.624) (width 0.127) (layer "F.Cu") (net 8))
 (segment (start 46.916901 48.624) (end 47.376 48.624) (width 0.127) (layer "F.Cu") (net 8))
 (segment (start 50.3 45.7) (end 50.3 44.82) (width 0.127) (layer "F.Cu") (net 8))
 (segment (start 46.7 49) (end 46.7 48.840901) (width 0.127) (layer "F.Cu") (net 8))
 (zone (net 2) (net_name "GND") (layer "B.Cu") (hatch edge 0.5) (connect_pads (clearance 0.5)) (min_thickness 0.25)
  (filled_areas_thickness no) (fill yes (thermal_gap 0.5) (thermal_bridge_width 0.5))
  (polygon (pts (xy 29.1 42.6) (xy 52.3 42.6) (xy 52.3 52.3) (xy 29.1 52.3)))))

